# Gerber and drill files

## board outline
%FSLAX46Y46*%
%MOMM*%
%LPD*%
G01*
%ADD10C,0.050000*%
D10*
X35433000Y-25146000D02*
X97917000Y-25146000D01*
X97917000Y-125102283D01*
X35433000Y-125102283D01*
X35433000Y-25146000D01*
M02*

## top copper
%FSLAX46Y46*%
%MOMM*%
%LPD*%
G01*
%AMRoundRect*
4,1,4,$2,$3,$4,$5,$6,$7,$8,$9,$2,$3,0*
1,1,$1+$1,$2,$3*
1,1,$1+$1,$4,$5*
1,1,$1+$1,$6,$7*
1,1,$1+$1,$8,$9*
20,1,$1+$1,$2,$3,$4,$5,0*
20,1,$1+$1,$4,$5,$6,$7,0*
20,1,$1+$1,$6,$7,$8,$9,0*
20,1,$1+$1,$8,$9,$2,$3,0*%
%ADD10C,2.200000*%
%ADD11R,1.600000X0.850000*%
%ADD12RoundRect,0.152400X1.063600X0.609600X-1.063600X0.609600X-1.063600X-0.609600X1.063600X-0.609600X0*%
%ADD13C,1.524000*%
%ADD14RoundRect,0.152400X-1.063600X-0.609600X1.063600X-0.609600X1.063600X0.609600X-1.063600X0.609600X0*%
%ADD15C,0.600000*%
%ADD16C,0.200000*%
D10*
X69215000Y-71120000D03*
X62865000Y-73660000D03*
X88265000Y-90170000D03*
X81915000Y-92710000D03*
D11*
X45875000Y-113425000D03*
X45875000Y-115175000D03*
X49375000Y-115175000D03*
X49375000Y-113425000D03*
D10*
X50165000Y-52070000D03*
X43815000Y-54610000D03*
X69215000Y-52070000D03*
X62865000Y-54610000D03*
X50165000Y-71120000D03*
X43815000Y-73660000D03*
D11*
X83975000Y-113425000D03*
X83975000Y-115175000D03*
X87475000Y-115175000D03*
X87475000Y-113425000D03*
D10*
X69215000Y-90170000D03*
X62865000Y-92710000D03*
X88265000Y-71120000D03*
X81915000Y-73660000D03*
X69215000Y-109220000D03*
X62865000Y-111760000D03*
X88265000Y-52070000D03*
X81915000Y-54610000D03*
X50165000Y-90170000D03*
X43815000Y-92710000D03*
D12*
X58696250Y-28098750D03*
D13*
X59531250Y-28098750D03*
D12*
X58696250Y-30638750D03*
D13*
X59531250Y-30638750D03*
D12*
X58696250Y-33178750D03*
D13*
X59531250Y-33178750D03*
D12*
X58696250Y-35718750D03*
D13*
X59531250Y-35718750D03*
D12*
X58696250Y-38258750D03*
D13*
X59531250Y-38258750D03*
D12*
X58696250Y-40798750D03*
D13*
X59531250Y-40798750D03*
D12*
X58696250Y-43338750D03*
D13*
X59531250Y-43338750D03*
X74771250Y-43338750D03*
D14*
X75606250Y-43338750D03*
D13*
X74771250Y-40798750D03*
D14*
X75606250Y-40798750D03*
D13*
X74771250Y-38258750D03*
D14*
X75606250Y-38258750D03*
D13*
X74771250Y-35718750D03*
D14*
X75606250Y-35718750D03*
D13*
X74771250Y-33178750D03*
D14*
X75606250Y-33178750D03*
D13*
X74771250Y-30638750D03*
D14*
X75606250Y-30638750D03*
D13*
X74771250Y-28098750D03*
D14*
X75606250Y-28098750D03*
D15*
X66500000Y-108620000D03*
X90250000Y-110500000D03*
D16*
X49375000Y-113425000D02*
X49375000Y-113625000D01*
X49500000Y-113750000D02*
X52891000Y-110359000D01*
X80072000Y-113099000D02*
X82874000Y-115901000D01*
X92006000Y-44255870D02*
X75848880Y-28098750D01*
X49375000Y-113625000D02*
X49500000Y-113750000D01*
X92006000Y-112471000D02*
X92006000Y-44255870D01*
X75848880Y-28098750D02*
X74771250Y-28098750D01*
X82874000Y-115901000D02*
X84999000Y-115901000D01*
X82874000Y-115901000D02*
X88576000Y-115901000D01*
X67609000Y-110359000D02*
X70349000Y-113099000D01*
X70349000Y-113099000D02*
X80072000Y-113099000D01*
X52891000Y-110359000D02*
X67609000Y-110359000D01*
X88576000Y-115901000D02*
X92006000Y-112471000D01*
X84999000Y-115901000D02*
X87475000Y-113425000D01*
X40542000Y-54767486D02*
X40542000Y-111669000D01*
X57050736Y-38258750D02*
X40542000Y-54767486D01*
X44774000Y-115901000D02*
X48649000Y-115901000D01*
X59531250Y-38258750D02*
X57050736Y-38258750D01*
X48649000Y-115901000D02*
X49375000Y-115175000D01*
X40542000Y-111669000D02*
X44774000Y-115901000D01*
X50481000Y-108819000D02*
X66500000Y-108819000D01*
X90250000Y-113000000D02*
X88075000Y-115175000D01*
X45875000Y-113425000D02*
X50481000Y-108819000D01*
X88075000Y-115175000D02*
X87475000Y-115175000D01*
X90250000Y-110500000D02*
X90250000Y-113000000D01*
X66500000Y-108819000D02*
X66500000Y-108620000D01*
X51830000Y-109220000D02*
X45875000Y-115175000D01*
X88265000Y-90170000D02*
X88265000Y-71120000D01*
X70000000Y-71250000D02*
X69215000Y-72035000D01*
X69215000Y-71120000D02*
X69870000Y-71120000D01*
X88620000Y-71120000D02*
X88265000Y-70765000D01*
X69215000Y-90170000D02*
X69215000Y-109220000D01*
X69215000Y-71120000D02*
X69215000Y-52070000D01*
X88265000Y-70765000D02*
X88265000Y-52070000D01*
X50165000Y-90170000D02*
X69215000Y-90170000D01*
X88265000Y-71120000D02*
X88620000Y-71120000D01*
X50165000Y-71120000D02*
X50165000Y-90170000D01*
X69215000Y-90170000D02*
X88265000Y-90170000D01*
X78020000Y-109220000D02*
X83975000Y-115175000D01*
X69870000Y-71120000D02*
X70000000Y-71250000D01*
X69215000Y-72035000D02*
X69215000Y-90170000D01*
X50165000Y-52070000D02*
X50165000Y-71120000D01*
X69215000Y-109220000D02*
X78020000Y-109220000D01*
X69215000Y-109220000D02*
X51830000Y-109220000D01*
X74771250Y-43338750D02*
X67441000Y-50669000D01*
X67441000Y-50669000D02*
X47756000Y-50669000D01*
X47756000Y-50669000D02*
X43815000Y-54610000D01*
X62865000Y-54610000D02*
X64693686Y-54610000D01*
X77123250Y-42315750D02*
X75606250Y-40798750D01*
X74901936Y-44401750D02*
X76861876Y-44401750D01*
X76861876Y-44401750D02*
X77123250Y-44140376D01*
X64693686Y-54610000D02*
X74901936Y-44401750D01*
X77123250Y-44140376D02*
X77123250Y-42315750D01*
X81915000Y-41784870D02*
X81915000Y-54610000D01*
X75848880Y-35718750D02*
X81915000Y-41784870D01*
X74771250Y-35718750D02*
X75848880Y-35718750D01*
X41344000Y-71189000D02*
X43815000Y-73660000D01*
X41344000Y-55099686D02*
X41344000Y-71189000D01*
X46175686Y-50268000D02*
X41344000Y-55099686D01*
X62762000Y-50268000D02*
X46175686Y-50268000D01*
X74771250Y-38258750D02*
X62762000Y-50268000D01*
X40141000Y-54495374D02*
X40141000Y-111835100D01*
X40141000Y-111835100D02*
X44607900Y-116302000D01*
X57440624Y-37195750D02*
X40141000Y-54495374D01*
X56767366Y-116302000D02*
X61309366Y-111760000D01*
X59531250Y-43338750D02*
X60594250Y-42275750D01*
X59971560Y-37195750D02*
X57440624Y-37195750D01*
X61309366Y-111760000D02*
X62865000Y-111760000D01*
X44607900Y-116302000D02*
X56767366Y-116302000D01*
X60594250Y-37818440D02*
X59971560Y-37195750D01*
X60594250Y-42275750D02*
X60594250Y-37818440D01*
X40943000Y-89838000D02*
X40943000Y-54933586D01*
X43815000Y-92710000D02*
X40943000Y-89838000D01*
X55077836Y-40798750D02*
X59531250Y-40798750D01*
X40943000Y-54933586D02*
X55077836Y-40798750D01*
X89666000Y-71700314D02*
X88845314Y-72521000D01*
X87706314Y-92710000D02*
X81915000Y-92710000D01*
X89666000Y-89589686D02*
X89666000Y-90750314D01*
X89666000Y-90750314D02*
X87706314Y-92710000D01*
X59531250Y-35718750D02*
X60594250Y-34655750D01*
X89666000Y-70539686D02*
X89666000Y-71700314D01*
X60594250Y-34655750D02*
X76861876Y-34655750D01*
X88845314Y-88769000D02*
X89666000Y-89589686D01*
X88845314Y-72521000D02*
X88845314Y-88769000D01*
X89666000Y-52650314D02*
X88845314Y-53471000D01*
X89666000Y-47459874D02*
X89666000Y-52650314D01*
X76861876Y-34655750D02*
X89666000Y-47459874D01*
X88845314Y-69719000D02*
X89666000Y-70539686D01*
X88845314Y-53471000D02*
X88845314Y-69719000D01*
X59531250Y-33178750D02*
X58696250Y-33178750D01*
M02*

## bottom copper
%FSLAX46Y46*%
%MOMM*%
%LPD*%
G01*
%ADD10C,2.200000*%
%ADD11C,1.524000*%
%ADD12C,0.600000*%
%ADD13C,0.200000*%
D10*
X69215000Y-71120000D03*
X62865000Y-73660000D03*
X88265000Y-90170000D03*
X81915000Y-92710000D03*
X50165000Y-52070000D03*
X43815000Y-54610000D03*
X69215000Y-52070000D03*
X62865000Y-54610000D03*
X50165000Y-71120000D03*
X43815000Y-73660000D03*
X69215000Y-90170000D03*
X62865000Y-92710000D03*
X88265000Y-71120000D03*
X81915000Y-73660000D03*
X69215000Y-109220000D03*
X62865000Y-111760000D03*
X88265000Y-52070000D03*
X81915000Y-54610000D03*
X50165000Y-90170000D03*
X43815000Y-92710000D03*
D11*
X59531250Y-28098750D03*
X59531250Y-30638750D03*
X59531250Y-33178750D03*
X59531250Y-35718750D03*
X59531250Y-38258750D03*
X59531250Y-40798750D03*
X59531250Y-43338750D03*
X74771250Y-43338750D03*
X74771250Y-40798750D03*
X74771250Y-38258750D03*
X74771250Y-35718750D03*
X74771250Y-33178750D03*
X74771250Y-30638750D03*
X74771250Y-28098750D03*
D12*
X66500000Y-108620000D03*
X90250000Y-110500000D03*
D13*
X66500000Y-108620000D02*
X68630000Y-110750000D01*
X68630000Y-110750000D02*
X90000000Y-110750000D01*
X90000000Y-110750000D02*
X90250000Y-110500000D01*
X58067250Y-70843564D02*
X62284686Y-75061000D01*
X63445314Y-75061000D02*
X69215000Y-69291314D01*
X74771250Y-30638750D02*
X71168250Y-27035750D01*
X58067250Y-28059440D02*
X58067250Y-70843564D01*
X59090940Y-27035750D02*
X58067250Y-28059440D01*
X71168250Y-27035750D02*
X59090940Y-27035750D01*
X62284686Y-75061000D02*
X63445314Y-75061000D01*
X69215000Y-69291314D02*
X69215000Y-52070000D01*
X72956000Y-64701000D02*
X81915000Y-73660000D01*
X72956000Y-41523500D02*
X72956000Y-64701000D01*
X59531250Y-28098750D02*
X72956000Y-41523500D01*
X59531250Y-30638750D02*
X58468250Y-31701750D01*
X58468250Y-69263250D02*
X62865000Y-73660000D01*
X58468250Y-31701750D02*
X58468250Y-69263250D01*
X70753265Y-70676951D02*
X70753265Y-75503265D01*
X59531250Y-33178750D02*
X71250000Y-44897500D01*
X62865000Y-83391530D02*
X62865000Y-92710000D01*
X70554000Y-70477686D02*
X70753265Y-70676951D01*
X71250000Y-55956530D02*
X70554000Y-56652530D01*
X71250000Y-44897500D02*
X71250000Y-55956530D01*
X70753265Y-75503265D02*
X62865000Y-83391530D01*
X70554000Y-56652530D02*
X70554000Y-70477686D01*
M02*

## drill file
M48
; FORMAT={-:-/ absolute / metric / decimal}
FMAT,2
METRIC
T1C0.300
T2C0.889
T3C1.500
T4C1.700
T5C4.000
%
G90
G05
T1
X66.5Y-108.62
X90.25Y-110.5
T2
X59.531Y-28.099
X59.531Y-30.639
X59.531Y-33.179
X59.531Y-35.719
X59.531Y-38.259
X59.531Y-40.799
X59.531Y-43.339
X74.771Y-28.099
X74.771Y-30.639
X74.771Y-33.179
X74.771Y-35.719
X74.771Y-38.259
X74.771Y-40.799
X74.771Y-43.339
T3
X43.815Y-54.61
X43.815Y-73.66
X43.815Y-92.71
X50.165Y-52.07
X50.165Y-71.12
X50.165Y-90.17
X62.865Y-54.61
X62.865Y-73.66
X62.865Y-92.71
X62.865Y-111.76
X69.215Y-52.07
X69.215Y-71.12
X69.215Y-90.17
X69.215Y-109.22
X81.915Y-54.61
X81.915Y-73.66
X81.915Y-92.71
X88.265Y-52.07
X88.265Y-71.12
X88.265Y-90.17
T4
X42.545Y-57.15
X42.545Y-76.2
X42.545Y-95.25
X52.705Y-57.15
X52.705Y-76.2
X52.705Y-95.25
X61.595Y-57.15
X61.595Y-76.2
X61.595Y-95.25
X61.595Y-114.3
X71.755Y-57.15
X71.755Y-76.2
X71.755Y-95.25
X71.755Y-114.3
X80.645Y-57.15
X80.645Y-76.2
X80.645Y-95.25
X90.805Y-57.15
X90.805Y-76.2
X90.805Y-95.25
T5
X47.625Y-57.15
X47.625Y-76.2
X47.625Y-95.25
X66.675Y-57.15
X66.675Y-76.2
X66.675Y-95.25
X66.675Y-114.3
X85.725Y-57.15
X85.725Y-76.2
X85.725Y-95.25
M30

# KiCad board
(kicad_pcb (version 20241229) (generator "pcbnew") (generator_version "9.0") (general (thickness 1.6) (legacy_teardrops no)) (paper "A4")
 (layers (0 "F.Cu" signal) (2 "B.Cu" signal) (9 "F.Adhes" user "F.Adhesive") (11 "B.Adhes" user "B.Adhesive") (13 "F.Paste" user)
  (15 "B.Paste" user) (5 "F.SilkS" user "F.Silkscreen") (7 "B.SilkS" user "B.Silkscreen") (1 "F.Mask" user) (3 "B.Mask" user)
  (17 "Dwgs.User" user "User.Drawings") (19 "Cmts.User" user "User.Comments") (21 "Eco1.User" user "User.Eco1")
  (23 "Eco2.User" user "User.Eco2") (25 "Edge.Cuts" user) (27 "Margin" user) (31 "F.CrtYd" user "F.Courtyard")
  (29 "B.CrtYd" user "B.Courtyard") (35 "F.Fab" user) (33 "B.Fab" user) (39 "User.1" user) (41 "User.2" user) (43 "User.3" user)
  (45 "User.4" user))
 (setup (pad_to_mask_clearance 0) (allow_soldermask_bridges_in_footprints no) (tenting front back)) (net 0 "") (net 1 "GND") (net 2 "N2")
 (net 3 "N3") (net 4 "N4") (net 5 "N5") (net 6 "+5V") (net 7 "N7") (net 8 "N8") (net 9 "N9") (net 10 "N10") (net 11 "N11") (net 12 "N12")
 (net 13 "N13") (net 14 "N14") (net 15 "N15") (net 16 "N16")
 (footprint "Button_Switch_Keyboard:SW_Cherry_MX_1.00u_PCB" (layer "F.Cu") (at 69.215 71.12)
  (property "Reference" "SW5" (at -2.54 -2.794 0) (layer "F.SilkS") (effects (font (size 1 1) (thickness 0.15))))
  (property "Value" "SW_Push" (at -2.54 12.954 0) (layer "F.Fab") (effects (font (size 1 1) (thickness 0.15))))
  (pad "" np_thru_hole circle (at -7.62 5.08) (size 1.7 1.7) (drill 1.7) (layers "*.Cu" "*.Mask"))
  (pad "" np_thru_hole circle (at -2.54 5.08) (size 4 4) (drill 4) (layers "*.Cu" "*.Mask"))
  (pad "" np_thru_hole circle (at 2.54 5.08) (size 1.7 1.7) (drill 1.7) (layers "*.Cu" "*.Mask"))
  (pad "1" thru_hole circle (at 0 0) (size 2.2 2.2) (drill 1.5) (layers "*.Cu" "*.Mask") (remove_unused_layers no) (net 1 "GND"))
  (pad "2" thru_hole circle (at -6.35 2.54) (size 2.2 2.2) (drill 1.5) (layers "*.Cu" "*.Mask") (remove_unused_layers no) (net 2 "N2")))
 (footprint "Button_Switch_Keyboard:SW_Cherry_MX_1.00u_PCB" (layer "F.Cu") (at 88.265 90.17)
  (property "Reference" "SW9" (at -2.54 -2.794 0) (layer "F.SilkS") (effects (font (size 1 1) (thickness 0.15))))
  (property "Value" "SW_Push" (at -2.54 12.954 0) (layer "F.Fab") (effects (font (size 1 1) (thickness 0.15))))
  (pad "" np_thru_hole circle (at -7.62 5.08) (size 1.7 1.7) (drill 1.7) (layers "*.Cu" "*.Mask"))
  (pad "" np_thru_hole circle (at -2.54 5.08) (size 4 4) (drill 4) (layers "*.Cu" "*.Mask"))
  (pad "" np_thru_hole circle (at 2.54 5.08) (size 1.7 1.7) (drill 1.7) (layers "*.Cu" "*.Mask"))
  (pad "1" thru_hole circle (at 0 0) (size 2.2 2.2) (drill 1.5) (layers "*.Cu" "*.Mask") (remove_unused_layers no) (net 1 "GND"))
  (pad "2" thru_hole circle (at -6.35 2.54) (size 2.2 2.2) (drill 1.5) (layers "*.Cu" "*.Mask") (remove_unused_layers no) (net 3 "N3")))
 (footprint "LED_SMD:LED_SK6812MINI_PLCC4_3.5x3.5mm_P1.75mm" (layer "F.Cu") (at 47.625 114.3)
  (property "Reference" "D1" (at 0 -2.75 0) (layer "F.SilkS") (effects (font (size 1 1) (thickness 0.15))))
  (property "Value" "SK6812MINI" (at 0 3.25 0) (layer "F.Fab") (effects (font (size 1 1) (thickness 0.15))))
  (pad "1" smd rect (at -1.75 -0.875) (size 1.6 0.85) (layers "F.Cu" "F.Mask" "F.Paste") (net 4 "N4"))
  (pad "2" smd rect (at -1.75 0.875) (size 1.6 0.85) (layers "F.Cu" "F.Mask" "F.Paste") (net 1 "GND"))
  (pad "3" smd rect (at 1.75 0.875) (size 1.6 0.85) (layers "F.Cu" "F.Mask" "F.Paste") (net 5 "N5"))
  (pad "4" smd rect (at 1.75 -0.875) (size 1.6 0.85) (layers "F.Cu" "F.Mask" "F.Paste") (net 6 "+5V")))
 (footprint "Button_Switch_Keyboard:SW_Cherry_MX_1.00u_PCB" (layer "F.Cu") (at 50.165 52.07)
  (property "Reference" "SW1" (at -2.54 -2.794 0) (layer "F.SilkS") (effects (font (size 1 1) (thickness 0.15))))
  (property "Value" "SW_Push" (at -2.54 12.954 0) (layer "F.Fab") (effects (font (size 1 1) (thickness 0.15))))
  (pad "" np_thru_hole circle (at -7.62 5.08) (size 1.7 1.7) (drill 1.7) (layers "*.Cu" "*.Mask"))
  (pad "" np_thru_hole circle (at -2.54 5.08) (size 4 4) (drill 4) (layers "*.Cu" "*.Mask"))
  (pad "" np_thru_hole circle (at 2.54 5.08) (size 1.7 1.7) (drill 1.7) (layers "*.Cu" "*.Mask"))
  (pad "1" thru_hole circle (at 0 0) (size 2.2 2.2) (drill 1.5) (layers "*.Cu" "*.Mask") (remove_unused_layers no) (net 1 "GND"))
  (pad "2" thru_hole circle (at -6.35 2.54) (size 2.2 2.2) (drill 1.5) (layers "*.Cu" "*.Mask") (remove_unused_layers no) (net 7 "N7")))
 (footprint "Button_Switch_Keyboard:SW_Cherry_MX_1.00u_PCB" (layer "F.Cu") (at 69.215 52.07)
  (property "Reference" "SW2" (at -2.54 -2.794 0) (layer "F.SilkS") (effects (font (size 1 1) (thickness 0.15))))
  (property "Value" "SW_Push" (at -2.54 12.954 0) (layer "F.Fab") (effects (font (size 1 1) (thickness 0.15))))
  (pad "" np_thru_hole circle (at -7.62 5.08) (size 1.7 1.7) (drill 1.7) (layers "*.Cu" "*.Mask"))
  (pad "" np_thru_hole circle (at -2.54 5.08) (size 4 4) (drill 4) (layers "*.Cu" "*.Mask"))
  (pad "" np_thru_hole circle (at 2.54 5.08) (size 1.7 1.7) (drill 1.7) (layers "*.Cu" "*.Mask"))
  (pad "1" thru_hole circle (at 0 0) (size 2.2 2.2) (drill 1.5) (layers "*.Cu" "*.Mask") (remove_unused_layers no) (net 1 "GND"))
  (pad "2" thru_hole circle (at -6.35 2.54) (size 2.2 2.2) (drill 1.5) (layers "*.Cu" "*.Mask") (remove_unused_layers no) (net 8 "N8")))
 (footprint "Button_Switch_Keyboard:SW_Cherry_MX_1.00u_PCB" (layer "F.Cu") (at 50.165 71.12)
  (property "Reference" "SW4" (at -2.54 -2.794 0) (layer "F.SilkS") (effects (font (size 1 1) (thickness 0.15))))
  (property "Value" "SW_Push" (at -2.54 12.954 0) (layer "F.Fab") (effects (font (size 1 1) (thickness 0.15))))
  (pad "" np_thru_hole circle (at -7.62 5.08) (size 1.7 1.7) (drill 1.7) (layers "*.Cu" "*.Mask"))
  (pad "" np_thru_hole circle (at -2.54 5.08) (size 4 4) (drill 4) (layers "*.Cu" "*.Mask"))
  (pad "" np_thru_hole circle (at 2.54 5.08) (size 1.7 1.7) (drill 1.7) (layers "*.Cu" "*.Mask"))
  (pad "1" thru_hole circle (at 0 0) (size 2.2 2.2) (drill 1.5) (layers "*.Cu" "*.Mask") (remove_unused_layers no) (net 1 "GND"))
  (pad "2" thru_hole circle (at -6.35 2.54) (size 2.2 2.2) (drill 1.5) (layers "*.Cu" "*.Mask") (remove_unused_layers no) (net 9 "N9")))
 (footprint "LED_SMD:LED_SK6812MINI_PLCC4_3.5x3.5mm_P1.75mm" (layer "F.Cu") (at 85.725 114.3)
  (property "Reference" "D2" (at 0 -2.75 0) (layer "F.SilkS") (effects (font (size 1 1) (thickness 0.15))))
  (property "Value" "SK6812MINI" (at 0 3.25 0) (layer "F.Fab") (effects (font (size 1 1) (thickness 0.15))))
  (pad "1" smd rect (at -1.75 -0.875) (size 1.6 0.85) (layers "F.Cu" "F.Mask" "F.Paste") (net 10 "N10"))
  (pad "2" smd rect (at -1.75 0.875) (size 1.6 0.85) (layers "F.Cu" "F.Mask" "F.Paste") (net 1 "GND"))
  (pad "3" smd rect (at 1.75 0.875) (size 1.6 0.85) (layers "F.Cu" "F.Mask" "F.Paste") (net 4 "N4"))
  (pad "4" smd rect (at 1.75 -0.875) (size 1.6 0.85) (layers "F.Cu" "F.Mask" "F.Paste") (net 6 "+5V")))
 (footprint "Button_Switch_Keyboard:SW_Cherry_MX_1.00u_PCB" (layer "F.Cu") (at 69.215 90.17)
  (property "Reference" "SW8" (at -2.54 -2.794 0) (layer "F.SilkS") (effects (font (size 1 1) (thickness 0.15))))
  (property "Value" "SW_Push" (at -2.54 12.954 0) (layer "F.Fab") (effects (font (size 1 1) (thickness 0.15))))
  (pad "" np_thru_hole circle (at -7.62 5.08) (size 1.7 1.7) (drill 1.7) (layers "*.Cu" "*.Mask"))
  (pad "" np_thru_hole circle (at -2.54 5.08) (size 4 4) (drill 4) (layers "*.Cu" "*.Mask"))
  (pad "" np_thru_hole circle (at 2.54 5.08) (size 1.7 1.7) (drill 1.7) (layers "*.Cu" "*.Mask"))
  (pad "1" thru_hole circle (at 0 0) (size 2.2 2.2) (drill 1.5) (layers "*.Cu" "*.Mask") (remove_unused_layers no) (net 1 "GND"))
  (pad "2" thru_hole circle (at -6.35 2.54) (size 2.2 2.2) (drill 1.5) (layers "*.Cu" "*.Mask") (remove_unused_layers no) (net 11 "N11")))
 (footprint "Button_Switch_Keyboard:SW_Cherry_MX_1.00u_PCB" (layer "F.Cu") (at 88.265 71.12)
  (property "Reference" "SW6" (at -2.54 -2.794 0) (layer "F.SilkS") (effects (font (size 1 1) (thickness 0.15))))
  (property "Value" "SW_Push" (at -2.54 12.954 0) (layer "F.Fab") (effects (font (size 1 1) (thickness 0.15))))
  (pad "" np_thru_hole circle (at -7.62 5.08) (size 1.7 1.7) (drill 1.7) (layers "*.Cu" "*.Mask"))
  (pad "" np_thru_hole circle (at -2.54 5.08) (size 4 4) (drill 4) (layers "*.Cu" "*.Mask"))
  (pad "" np_thru_hole circle (at 2.54 5.08) (size 1.7 1.7) (drill 1.7) (layers "*.Cu" "*.Mask"))
  (pad "1" thru_hole circle (at 0 0) (size 2.2 2.2) (drill 1.5) (layers "*.Cu" "*.Mask") (remove_unused_layers no) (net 1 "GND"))
  (pad "2" thru_hole circle (at -6.35 2.54) (size 2.2 2.2) (drill 1.5) (layers "*.Cu" "*.Mask") (remove_unused_layers no) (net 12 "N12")))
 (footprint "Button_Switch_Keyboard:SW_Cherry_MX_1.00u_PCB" (layer "F.Cu") (at 69.215 109.22)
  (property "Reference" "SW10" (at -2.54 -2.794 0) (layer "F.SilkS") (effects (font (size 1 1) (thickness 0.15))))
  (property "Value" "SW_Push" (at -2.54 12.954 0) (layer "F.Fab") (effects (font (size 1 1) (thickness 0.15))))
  (pad "" np_thru_hole circle (at -7.62 5.08) (size 1.7 1.7) (drill 1.7) (layers "*.Cu" "*.Mask"))
  (pad "" np_thru_hole circle (at -2.54 5.08) (size 4 4) (drill 4) (layers "*.Cu" "*.Mask"))
  (pad "" np_thru_hole circle (at 2.54 5.08) (size 1.7 1.7) (drill 1.7) (layers "*.Cu" "*.Mask"))
  (pad "1" thru_hole circle (at 0 0) (size 2.2 2.2) (drill 1.5) (layers "*.Cu" "*.Mask") (remove_unused_layers no) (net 1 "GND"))
  (pad "2" thru_hole circle (at -6.35 2.54) (size 2.2 2.2) (drill 1.5) (layers "*.Cu" "*.Mask") (remove_unused_layers no) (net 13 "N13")))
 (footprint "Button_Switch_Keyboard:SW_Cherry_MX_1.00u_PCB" (layer "F.Cu") (at 88.265 52.07)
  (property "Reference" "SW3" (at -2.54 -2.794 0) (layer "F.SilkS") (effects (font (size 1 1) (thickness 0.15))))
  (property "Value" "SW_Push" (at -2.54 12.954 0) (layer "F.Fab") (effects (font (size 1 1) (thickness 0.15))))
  (pad "" np_thru_hole circle (at -7.62 5.08) (size 1.7 1.7) (drill 1.7) (layers "*.Cu" "*.Mask"))
  (pad "" np_thru_hole circle (at -2.54 5.08) (size 4 4) (drill 4) (layers "*.Cu" "*.Mask"))
  (pad "" np_thru_hole circle (at 2.54 5.08) (size 1.7 1.7) (drill 1.7) (layers "*.Cu" "*.Mask"))
  (pad "1" thru_hole circle (at 0 0) (size 2.2 2.2) (drill 1.5) (layers "*.Cu" "*.Mask") (remove_unused_layers no) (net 1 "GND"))
  (pad "2" thru_hole circle (at -6.35 2.54) (size 2.2 2.2) (drill 1.5) (layers "*.Cu" "*.Mask") (remove_unused_layers no) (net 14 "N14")))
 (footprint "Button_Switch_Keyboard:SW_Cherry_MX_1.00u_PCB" (layer "F.Cu") (at 50.165 90.17)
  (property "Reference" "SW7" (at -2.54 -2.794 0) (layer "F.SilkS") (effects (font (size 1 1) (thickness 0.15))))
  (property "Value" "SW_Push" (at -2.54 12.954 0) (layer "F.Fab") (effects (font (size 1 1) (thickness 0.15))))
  (pad "" np_thru_hole circle (at -7.62 5.08) (size 1.7 1.7) (drill 1.7) (layers "*.Cu" "*.Mask"))
  (pad "" np_thru_hole circle (at -2.54 5.08) (size 4 4) (drill 4) (layers "*.Cu" "*.Mask"))
  (pad "" np_thru_hole circle (at 2.54 5.08) (size 1.7 1.7) (drill 1.7) (layers "*.Cu" "*.Mask"))
  (pad "1" thru_hole circle (at 0 0) (size 2.2 2.2) (drill 1.5) (layers "*.Cu" "*.Mask") (remove_unused_layers no) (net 1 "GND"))
  (pad "2" thru_hole circle (at -6.35 2.54) (size 2.2 2.2) (drill 1.5) (layers "*.Cu" "*.Mask") (remove_unused_layers no) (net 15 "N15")))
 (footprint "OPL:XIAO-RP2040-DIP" (layer "F.Cu") (at 67.15125 35.71875)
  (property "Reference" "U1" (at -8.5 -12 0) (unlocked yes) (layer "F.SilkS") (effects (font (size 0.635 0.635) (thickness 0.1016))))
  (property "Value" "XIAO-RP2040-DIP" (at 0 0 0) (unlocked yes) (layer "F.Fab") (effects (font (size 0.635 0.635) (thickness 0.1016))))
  (pad "1" smd roundrect (at -8.455 -7.62 180) (size 2.432 1.524) (layers "F.Cu" "F.Mask") (roundrect_rratio 0.1) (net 12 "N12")
   (thermal_bridge_angle 45))
  (pad "1" thru_hole circle (at -7.62 -7.62 180) (size 1.524 1.524) (drill 0.889) (layers "*.Cu" "*.Mask") (remove_unused_layers no)
   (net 12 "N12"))
  (pad "2" smd roundrect (at -8.455 -5.08 180) (size 2.432 1.524) (layers "F.Cu" "F.Mask") (roundrect_rratio 0.1) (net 2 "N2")
   (thermal_bridge_angle 45))
  (pad "2" thru_hole circle (at -7.62 -5.08 180) (size 1.524 1.524) (drill 0.889) (layers "*.Cu" "*.Mask") (remove_unused_layers no)
   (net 2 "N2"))
  (pad "3" smd roundrect (at -8.455 -2.54 180) (size 2.432 1.524) (layers "F.Cu" "F.Mask") (roundrect_rratio 0.1) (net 11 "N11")
   (thermal_bridge_angle 45))
  (pad "3" thru_hole circle (at -7.62 -2.54 180) (size 1.524 1.524) (drill 0.889) (layers "*.Cu" "*.Mask") (remove_unused_layers no)
   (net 11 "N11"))
  (pad "4" smd roundrect (at -8.455 0 180) (size 2.432 1.524) (layers "F.Cu" "F.Mask") (roundrect_rratio 0.1) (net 3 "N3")
   (thermal_bridge_angle 45))
  (pad "4" thru_hole circle (at -7.62 0 180) (size 1.524 1.524) (drill 0.889) (layers "*.Cu" "*.Mask") (remove_unused_layers no)
   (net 3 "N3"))
  (pad "5" smd roundrect (at -8.455 2.54 180) (size 2.432 1.524) (layers "F.Cu" "F.Mask") (roundrect_rratio 0.1) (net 5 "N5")
   (thermal_bridge_angle 45))
  (pad "5" thru_hole circle (at -7.62 2.54 180) (size 1.524 1.524) (drill 0.889) (layers "*.Cu" "*.Mask") (remove_unused_layers no)
   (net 5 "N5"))
  (pad "6" smd roundrect (at -8.455 5.08 180) (size 2.432 1.524) (layers "F.Cu" "F.Mask") (roundrect_rratio 0.1) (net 15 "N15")
   (thermal_bridge_angle 45))
  (pad "6" thru_hole circle (at -7.62 5.08 180) (size 1.524 1.524) (drill 0.889) (layers "*.Cu" "*.Mask") (remove_unused_layers no)
   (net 15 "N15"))
  (pad "7" smd roundrect (at -8.455 7.62 180) (size 2.432 1.524) (layers "F.Cu" "F.Mask") (roundrect_rratio 0.1) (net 13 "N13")
   (thermal_bridge_angle 45))
  (pad "7" thru_hole circle (at -7.62 7.62 180) (size 1.524 1.524) (drill 0.889) (layers "*.Cu" "*.Mask") (remove_unused_layers no)
   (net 13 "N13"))
  (pad "8" thru_hole circle (at 7.62 7.62) (size 1.524 1.524) (drill 0.889) (layers "*.Cu" "*.Mask") (remove_unused_layers no) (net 7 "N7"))
  (pad "8" smd roundrect (at 8.455 7.62) (size 2.432 1.524) (layers "F.Cu" "F.Mask") (roundrect_rratio 0.1) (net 7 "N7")
   (thermal_bridge_angle 45))
  (pad "9" thru_hole circle (at 7.62 5.08) (size 1.524 1.524) (drill 0.889) (layers "*.Cu" "*.Mask") (remove_unused_layers no) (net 8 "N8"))
  (pad "9" smd roundrect (at 8.455 5.08) (size 2.432 1.524) (layers "F.Cu" "F.Mask") (roundrect_rratio 0.1) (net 8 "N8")
   (thermal_bridge_angle 45))
  (pad "10" thru_hole circle (at 7.62 2.54) (size 1.524 1.524) (drill 0.889) (layers "*.Cu" "*.Mask") (remove_unused_layers no) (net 9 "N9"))
  (pad "10" smd roundrect (at 8.455 2.54) (size 2.432 1.524) (layers "F.Cu" "F.Mask") (roundrect_rratio 0.1) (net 9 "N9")
   (thermal_bridge_angle 45))
  (pad "11" thru_hole circle (at 7.62 0) (size 1.524 1.524) (drill 0.889) (layers "*.Cu" "*.Mask") (remove_unused_layers no) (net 14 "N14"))
  (pad "11" smd roundrect (at 8.455 0) (size 2.432 1.524) (layers "F.Cu" "F.Mask") (roundrect_rratio 0.1) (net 14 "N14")
   (thermal_bridge_angle 45))
  (pad "12" thru_hole circle (at 7.62 -2.54) (size 1.524 1.524) (drill 0.889) (layers "*.Cu" "*.Mask") (remove_unused_layers no)
   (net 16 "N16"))
  (pad "12" smd roundrect (at 8.455 -2.54) (size 2.432 1.524) (layers "F.Cu" "F.Mask") (roundrect_rratio 0.1) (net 16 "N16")
   (thermal_bridge_angle 45))
  (pad "13" thru_hole circle (at 7.62 -5.08) (size 1.524 1.524) (drill 0.889) (layers "*.Cu" "*.Mask") (remove_unused_layers no)
   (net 1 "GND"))
  (pad "13" smd roundrect (at 8.455 -5.08) (size 2.432 1.524) (layers "F.Cu" "F.Mask") (roundrect_rratio 0.1) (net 1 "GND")
   (thermal_bridge_angle 45))
  (pad "14" thru_hole circle (at 7.62 -7.62) (size 1.524 1.524) (drill 0.889) (layers "*.Cu" "*.Mask") (remove_unused_layers no)
   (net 6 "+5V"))
  (pad "14" smd roundrect (at 8.455 -7.62) (size 2.432 1.524) (layers "F.Cu" "F.Mask") (roundrect_rratio 0.1) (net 6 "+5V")
   (thermal_bridge_angle 45)))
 (gr_rect (start 35.433 25.146) (end 97.917 125.102283) (stroke (width 0.05) (type solid)) (fill no) (layer "Edge.Cuts"))
 (segment (start 49.375 113.425) (end 49.375 113.625) (width 0.2) (layer "F.Cu") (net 6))
 (segment (start 49.5 113.75) (end 52.891 110.359) (width 0.2) (layer "F.Cu") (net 6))
 (segment (start 80.072 113.099) (end 82.874 115.901) (width 0.2) (layer "F.Cu") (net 6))
 (segment (start 92.006 44.25587) (end 75.84888 28.09875) (width 0.2) (layer "F.Cu") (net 6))
 (segment (start 49.375 113.625) (end 49.5 113.75) (width 0.2) (layer "F.Cu") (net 6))
 (segment (start 92.006 112.471) (end 92.006 44.25587) (width 0.2) (layer "F.Cu") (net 6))
 (segment (start 75.84888 28.09875) (end 74.77125 28.09875) (width 0.2) (layer "F.Cu") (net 6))
 (segment (start 82.874 115.901) (end 84.999 115.901) (width 0.2) (layer "F.Cu") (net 6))
 (segment (start 82.874 115.901) (end 88.576 115.901) (width 0.2) (layer "F.Cu") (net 6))
 (segment (start 67.609 110.359) (end 70.349 113.099) (width 0.2) (layer "F.Cu") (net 6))
 (segment (start 70.349 113.099) (end 80.072 113.099) (width 0.2) (layer "F.Cu") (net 6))
 (segment (start 52.891 110.359) (end 67.609 110.359) (width 0.2) (layer "F.Cu") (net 6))
 (segment (start 88.576 115.901) (end 92.006 112.471) (width 0.2) (layer "F.Cu") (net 6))
 (segment (start 84.999 115.901) (end 87.475 113.425) (width 0.2) (layer "F.Cu") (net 6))
 (segment (start 40.542 54.767486) (end 40.542 111.669) (width 0.2) (layer "F.Cu") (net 5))
 (segment (start 57.050736 38.25875) (end 40.542 54.767486) (width 0.2) (layer "F.Cu") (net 5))
 (segment (start 44.774 115.901) (end 48.649 115.901) (width 0.2) (layer "F.Cu") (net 5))
 (segment (start 59.53125 38.25875) (end 57.050736 38.25875) (width 0.2) (layer "F.Cu") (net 5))
 (segment (start 48.649 115.901) (end 49.375 115.175) (width 0.2) (layer "F.Cu") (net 5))
 (segment (start 40.542 111.669) (end 44.774 115.901) (width 0.2) (layer "F.Cu") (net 5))
 (segment (start 50.481 108.819) (end 66.5 108.819) (width 0.2) (layer "F.Cu") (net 4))
 (segment (start 90.25 113) (end 88.075 115.175) (width 0.2) (layer "F.Cu") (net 4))
 (segment (start 45.875 113.425) (end 50.481 108.819) (width 0.2) (layer "F.Cu") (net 4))
 (segment (start 88.075 115.175) (end 87.475 115.175) (width 0.2) (layer "F.Cu") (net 4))
 (segment (start 90.25 110.5) (end 90.25 113) (width 0.2) (layer "F.Cu") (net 4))
 (segment (start 66.5 108.819) (end 66.5 108.62) (width 0.2) (layer "F.Cu") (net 4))
 (via (at 66.5 108.62) (size 0.6) (drill 0.3) (layers "F.Cu" "B.Cu") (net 4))
 (via (at 90.25 110.5) (size 0.6) (drill 0.3) (layers "F.Cu" "B.Cu") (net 4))
 (segment (start 66.5 108.62) (end 68.63 110.75) (width 0.2) (layer "B.Cu") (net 4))
 (segment (start 68.63 110.75) (end 90 110.75) (width 0.2) (layer "B.Cu") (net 4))
 (segment (start 90 110.75) (end 90.25 110.5) (width 0.2) (layer "B.Cu") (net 4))
 (segment (start 51.83 109.22) (end 45.875 115.175) (width 0.2) (layer "F.Cu") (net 1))
 (segment (start 88.265 90.17) (end 88.265 71.12) (width 0.2) (layer "F.Cu") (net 1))
 (segment (start 70 71.25) (end 69.215 72.035) (width 0.2) (layer "F.Cu") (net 1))
 (segment (start 69.215 71.12) (end 69.87 71.12) (width 0.2) (layer "F.Cu") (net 1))
 (segment (start 88.62 71.12) (end 88.265 70.765) (width 0.2) (layer "F.Cu") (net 1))
 (segment (start 69.215 90.17) (end 69.215 109.22) (width 0.2) (layer "F.Cu") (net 1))
 (segment (start 69.215 71.12) (end 69.215 52.07) (width 0.2) (layer "F.Cu") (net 1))
 (segment (start 88.265 70.765) (end 88.265 52.07) (width 0.2) (layer "F.Cu") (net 1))
 (segment (start 50.165 90.17) (end 69.215 90.17) (width 0.2) (layer "F.Cu") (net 1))
 (segment (start 88.265 71.12) (end 88.62 71.12) (width 0.2) (layer "F.Cu") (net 1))
 (segment (start 50.165 71.12) (end 50.165 90.17) (width 0.2) (layer "F.Cu") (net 1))
 (segment (start 69.215 90.17) (end 88.265 90.17) (width 0.2) (layer "F.Cu") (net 1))
 (segment (start 78.02 109.22) (end 83.975 115.175) (width 0.2) (layer "F.Cu") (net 1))
 (segment (start 69.87 71.12) (end 70 71.25) (width 0.2) (layer "F.Cu") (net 1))
 (segment (start 69.215 72.035) (end 69.215 90.17) (width 0.2) (layer "F.Cu") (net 1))
 (segment (start 50.165 52.07) (end 50.165 71.12) (width 0.2) (layer "F.Cu") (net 1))
 (segment (start 69.215 109.22) (end 78.02 109.22) (width 0.2) (layer "F.Cu") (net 1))
 (segment (start 69.215 109.22) (end 51.83 109.22) (width 0.2) (layer "F.Cu") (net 1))
 (segment (start 58.06725 70.843564) (end 62.284686 75.061) (width 0.2) (layer "B.Cu") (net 1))
 (segment (start 63.445314 75.061) (end 69.215 69.291314) (width 0.2) (layer "B.Cu") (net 1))
 (segment (start 74.77125 30.63875) (end 71.16825 27.03575) (width 0.2) (layer "B.Cu") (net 1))
 (segment (start 58.06725 28.05944) (end 58.06725 70.843564) (width 0.2) (layer "B.Cu") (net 1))
 (segment (start 59.09094 27.03575) (end 58.06725 28.05944) (width 0.2) (layer "B.Cu") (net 1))
 (segment (start 71.16825 27.03575) (end 59.09094 27.03575) (width 0.2) (layer "B.Cu") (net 1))
 (segment (start 62.284686 75.061) (end 63.445314 75.061) (width 0.2) (layer "B.Cu") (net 1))
 (segment (start 69.215 69.291314) (end 69.215 52.07) (width 0.2) (layer "B.Cu") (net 1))
 (segment (start 74.77125 43.33875) (end 67.441 50.669) (width 0.2) (layer "F.Cu") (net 7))
 (segment (start 67.441 50.669) (end 47.756 50.669) (width 0.2) (layer "F.Cu") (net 7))
 (segment (start 47.756 50.669) (end 43.815 54.61) (width 0.2) (layer "F.Cu") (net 7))
 (segment (start 62.865 54.61) (end 64.693686 54.61) (width 0.2) (layer "F.Cu") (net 8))
 (segment (start 77.12325 42.31575) (end 75.60625 40.79875) (width 0.2) (layer "F.Cu") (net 8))
 (segment (start 74.901936 44.40175) (end 76.861876 44.40175) (width 0.2) (layer "F.Cu") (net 8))
 (segment (start 76.861876 44.40175) (end 77.12325 44.140376) (width 0.2) (layer "F.Cu") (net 8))
 (segment (start 64.693686 54.61) (end 74.901936 44.40175) (width 0.2) (layer "F.Cu") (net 8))
 (segment (start 77.12325 44.140376) (end 77.12325 42.31575) (width 0.2) (layer "F.Cu") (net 8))
 (segment (start 81.915 41.78487) (end 81.915 54.61) (width 0.2) (layer "F.Cu") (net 14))
 (segment (start 75.84888 35.71875) (end 81.915 41.78487) (width 0.2) (layer "F.Cu") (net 14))
 (segment (start 74.77125 35.71875) (end 75.84888 35.71875) (width 0.2) (layer "F.Cu") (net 14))
 (segment (start 41.344 71.189) (end 43.815 73.66) (width 0.2) (layer "F.Cu") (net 9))
 (segment (start 41.344 55.099686) (end 41.344 71.189) (width 0.2) (layer "F.Cu") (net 9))
 (segment (start 46.175686 50.268) (end 41.344 55.099686) (width 0.2) (layer "F.Cu") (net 9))
 (segment (start 62.762 50.268) (end 46.175686 50.268) (width 0.2) (layer "F.Cu") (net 9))
 (segment (start 74.77125 38.25875) (end 62.762 50.268) (width 0.2) (layer "F.Cu") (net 9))
 (segment (start 40.141 54.495374) (end 40.141 111.8351) (width 0.2) (layer "F.Cu") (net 13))
 (segment (start 40.141 111.8351) (end 44.6079 116.302) (width 0.2) (layer "F.Cu") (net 13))
 (segment (start 57.440624 37.19575) (end 40.141 54.495374) (width 0.2) (layer "F.Cu") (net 13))
 (segment (start 56.767366 116.302) (end 61.309366 111.76) (width 0.2) (layer "F.Cu") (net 13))
 (segment (start 59.53125 43.33875) (end 60.59425 42.27575) (width 0.2) (layer "F.Cu") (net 13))
 (segment (start 59.97156 37.19575) (end 57.440624 37.19575) (width 0.2) (layer "F.Cu") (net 13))
 (segment (start 61.309366 111.76) (end 62.865 111.76) (width 0.2) (layer "F.Cu") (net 13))
 (segment (start 44.6079 116.302) (end 56.767366 116.302) (width 0.2) (layer "F.Cu") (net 13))
 (segment (start 60.59425 37.81844) (end 59.97156 37.19575) (width 0.2) (layer "F.Cu") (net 13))
 (segment (start 60.59425 42.27575) (end 60.59425 37.81844) (width 0.2) (layer "F.Cu") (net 13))
 (segment (start 72.956 64.701) (end 81.915 73.66) (width 0.2) (layer "B.Cu") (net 12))
 (segment (start 72.956 41.5235) (end 72.956 64.701) (width 0.2) (layer "B.Cu") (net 12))
 (segment (start 59.53125 28.09875) (end 72.956 41.5235) (width 0.2) (layer "B.Cu") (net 12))
 (segment (start 40.943 89.838) (end 40.943 54.933586) (width 0.2) (layer "F.Cu") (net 15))
 (segment (start 43.815 92.71) (end 40.943 89.838) (width 0.2) (layer "F.Cu") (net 15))
 (segment (start 55.077836 40.79875) (end 59.53125 40.79875) (width 0.2) (layer "F.Cu") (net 15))
 (segment (start 40.943 54.933586) (end 55.077836 40.79875) (width 0.2) (layer "F.Cu") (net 15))
 (segment (start 89.666 71.700314) (end 88.845314 72.521) (width 0.2) (layer "F.Cu") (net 3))
 (segment (start 87.706314 92.71) (end 81.915 92.71) (width 0.2) (layer "F.Cu") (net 3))
 (segment (start 89.666 89.589686) (end 89.666 90.750314) (width 0.2) (layer "F.Cu") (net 3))
 (segment (start 89.666 90.750314) (end 87.706314 92.71) (width 0.2) (layer "F.Cu") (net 3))
 (segment (start 59.53125 35.71875) (end 60.59425 34.65575) (width 0.2) (layer "F.Cu") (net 3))
 (segment (start 89.666 70.539686) (end 89.666 71.700314) (width 0.2) (layer "F.Cu") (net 3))
 (segment (start 60.59425 34.65575) (end 76.861876 34.65575) (width 0.2) (layer "F.Cu") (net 3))
 (segment (start 88.845314 88.769) (end 89.666 89.589686) (width 0.2) (layer "F.Cu") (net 3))
 (segment (start 88.845314 72.521) (end 88.845314 88.769) (width 0.2) (layer "F.Cu") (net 3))
 (segment (start 89.666 52.650314) (end 88.845314 53.471) (width 0.2) (layer "F.Cu") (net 3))
 (segment (start 89.666 47.459874) (end 89.666 52.650314) (width 0.2) (layer "F.Cu") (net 3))
 (segment (start 76.861876 34.65575) (end 89.666 47.459874) (width 0.2) (layer "F.Cu") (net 3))
 (segment (start 88.845314 69.719) (end 89.666 70.539686) (width 0.2) (layer "F.Cu") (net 3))
 (segment (start 88.845314 53.471) (end 88.845314 69.719) (width 0.2) (layer "F.Cu") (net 3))
 (segment (start 59.53125 30.63875) (end 58.46825 31.70175) (width 0.2) (layer "B.Cu") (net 2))
 (segment (start 58.46825 69.26325) (end 62.865 73.66) (width 0.2) (layer "B.Cu") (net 2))
 (segment (start 58.46825 31.70175) (end 58.46825 69.26325) (width 0.2) (layer "B.Cu") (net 2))
 (segment (start 59.53125 33.17875) (end 58.69625 33.17875) (width 0.2) (layer "F.Cu") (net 11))
 (segment (start 70.753265 70.676951) (end 70.753265 75.503265) (width 0.2) (layer "B.Cu") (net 11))
 (segment (start 59.53125 33.17875) (end 71.25 44.8975) (width 0.2) (layer "B.Cu") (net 11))
 (segment (start 62.865 83.39153) (end 62.865 92.71) (width 0.2) (layer "B.Cu") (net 11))
 (segment (start 70.554 70.477686) (end 70.753265 70.676951) (width 0.2) (layer "B.Cu") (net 11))
 (segment (start 71.25 55.95653) (end 70.554 56.65253) (width 0.2) (layer "B.Cu") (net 11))
 (segment (start 71.25 44.8975) (end 71.25 55.95653) (width 0.2) (layer "B.Cu") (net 11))
 (segment (start 70.753265 75.503265) (end 62.865 83.39153) (width 0.2) (layer "B.Cu") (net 11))
 (segment (start 70.554 56.65253) (end 70.554 70.477686) (width 0.2) (layer "B.Cu") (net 11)))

